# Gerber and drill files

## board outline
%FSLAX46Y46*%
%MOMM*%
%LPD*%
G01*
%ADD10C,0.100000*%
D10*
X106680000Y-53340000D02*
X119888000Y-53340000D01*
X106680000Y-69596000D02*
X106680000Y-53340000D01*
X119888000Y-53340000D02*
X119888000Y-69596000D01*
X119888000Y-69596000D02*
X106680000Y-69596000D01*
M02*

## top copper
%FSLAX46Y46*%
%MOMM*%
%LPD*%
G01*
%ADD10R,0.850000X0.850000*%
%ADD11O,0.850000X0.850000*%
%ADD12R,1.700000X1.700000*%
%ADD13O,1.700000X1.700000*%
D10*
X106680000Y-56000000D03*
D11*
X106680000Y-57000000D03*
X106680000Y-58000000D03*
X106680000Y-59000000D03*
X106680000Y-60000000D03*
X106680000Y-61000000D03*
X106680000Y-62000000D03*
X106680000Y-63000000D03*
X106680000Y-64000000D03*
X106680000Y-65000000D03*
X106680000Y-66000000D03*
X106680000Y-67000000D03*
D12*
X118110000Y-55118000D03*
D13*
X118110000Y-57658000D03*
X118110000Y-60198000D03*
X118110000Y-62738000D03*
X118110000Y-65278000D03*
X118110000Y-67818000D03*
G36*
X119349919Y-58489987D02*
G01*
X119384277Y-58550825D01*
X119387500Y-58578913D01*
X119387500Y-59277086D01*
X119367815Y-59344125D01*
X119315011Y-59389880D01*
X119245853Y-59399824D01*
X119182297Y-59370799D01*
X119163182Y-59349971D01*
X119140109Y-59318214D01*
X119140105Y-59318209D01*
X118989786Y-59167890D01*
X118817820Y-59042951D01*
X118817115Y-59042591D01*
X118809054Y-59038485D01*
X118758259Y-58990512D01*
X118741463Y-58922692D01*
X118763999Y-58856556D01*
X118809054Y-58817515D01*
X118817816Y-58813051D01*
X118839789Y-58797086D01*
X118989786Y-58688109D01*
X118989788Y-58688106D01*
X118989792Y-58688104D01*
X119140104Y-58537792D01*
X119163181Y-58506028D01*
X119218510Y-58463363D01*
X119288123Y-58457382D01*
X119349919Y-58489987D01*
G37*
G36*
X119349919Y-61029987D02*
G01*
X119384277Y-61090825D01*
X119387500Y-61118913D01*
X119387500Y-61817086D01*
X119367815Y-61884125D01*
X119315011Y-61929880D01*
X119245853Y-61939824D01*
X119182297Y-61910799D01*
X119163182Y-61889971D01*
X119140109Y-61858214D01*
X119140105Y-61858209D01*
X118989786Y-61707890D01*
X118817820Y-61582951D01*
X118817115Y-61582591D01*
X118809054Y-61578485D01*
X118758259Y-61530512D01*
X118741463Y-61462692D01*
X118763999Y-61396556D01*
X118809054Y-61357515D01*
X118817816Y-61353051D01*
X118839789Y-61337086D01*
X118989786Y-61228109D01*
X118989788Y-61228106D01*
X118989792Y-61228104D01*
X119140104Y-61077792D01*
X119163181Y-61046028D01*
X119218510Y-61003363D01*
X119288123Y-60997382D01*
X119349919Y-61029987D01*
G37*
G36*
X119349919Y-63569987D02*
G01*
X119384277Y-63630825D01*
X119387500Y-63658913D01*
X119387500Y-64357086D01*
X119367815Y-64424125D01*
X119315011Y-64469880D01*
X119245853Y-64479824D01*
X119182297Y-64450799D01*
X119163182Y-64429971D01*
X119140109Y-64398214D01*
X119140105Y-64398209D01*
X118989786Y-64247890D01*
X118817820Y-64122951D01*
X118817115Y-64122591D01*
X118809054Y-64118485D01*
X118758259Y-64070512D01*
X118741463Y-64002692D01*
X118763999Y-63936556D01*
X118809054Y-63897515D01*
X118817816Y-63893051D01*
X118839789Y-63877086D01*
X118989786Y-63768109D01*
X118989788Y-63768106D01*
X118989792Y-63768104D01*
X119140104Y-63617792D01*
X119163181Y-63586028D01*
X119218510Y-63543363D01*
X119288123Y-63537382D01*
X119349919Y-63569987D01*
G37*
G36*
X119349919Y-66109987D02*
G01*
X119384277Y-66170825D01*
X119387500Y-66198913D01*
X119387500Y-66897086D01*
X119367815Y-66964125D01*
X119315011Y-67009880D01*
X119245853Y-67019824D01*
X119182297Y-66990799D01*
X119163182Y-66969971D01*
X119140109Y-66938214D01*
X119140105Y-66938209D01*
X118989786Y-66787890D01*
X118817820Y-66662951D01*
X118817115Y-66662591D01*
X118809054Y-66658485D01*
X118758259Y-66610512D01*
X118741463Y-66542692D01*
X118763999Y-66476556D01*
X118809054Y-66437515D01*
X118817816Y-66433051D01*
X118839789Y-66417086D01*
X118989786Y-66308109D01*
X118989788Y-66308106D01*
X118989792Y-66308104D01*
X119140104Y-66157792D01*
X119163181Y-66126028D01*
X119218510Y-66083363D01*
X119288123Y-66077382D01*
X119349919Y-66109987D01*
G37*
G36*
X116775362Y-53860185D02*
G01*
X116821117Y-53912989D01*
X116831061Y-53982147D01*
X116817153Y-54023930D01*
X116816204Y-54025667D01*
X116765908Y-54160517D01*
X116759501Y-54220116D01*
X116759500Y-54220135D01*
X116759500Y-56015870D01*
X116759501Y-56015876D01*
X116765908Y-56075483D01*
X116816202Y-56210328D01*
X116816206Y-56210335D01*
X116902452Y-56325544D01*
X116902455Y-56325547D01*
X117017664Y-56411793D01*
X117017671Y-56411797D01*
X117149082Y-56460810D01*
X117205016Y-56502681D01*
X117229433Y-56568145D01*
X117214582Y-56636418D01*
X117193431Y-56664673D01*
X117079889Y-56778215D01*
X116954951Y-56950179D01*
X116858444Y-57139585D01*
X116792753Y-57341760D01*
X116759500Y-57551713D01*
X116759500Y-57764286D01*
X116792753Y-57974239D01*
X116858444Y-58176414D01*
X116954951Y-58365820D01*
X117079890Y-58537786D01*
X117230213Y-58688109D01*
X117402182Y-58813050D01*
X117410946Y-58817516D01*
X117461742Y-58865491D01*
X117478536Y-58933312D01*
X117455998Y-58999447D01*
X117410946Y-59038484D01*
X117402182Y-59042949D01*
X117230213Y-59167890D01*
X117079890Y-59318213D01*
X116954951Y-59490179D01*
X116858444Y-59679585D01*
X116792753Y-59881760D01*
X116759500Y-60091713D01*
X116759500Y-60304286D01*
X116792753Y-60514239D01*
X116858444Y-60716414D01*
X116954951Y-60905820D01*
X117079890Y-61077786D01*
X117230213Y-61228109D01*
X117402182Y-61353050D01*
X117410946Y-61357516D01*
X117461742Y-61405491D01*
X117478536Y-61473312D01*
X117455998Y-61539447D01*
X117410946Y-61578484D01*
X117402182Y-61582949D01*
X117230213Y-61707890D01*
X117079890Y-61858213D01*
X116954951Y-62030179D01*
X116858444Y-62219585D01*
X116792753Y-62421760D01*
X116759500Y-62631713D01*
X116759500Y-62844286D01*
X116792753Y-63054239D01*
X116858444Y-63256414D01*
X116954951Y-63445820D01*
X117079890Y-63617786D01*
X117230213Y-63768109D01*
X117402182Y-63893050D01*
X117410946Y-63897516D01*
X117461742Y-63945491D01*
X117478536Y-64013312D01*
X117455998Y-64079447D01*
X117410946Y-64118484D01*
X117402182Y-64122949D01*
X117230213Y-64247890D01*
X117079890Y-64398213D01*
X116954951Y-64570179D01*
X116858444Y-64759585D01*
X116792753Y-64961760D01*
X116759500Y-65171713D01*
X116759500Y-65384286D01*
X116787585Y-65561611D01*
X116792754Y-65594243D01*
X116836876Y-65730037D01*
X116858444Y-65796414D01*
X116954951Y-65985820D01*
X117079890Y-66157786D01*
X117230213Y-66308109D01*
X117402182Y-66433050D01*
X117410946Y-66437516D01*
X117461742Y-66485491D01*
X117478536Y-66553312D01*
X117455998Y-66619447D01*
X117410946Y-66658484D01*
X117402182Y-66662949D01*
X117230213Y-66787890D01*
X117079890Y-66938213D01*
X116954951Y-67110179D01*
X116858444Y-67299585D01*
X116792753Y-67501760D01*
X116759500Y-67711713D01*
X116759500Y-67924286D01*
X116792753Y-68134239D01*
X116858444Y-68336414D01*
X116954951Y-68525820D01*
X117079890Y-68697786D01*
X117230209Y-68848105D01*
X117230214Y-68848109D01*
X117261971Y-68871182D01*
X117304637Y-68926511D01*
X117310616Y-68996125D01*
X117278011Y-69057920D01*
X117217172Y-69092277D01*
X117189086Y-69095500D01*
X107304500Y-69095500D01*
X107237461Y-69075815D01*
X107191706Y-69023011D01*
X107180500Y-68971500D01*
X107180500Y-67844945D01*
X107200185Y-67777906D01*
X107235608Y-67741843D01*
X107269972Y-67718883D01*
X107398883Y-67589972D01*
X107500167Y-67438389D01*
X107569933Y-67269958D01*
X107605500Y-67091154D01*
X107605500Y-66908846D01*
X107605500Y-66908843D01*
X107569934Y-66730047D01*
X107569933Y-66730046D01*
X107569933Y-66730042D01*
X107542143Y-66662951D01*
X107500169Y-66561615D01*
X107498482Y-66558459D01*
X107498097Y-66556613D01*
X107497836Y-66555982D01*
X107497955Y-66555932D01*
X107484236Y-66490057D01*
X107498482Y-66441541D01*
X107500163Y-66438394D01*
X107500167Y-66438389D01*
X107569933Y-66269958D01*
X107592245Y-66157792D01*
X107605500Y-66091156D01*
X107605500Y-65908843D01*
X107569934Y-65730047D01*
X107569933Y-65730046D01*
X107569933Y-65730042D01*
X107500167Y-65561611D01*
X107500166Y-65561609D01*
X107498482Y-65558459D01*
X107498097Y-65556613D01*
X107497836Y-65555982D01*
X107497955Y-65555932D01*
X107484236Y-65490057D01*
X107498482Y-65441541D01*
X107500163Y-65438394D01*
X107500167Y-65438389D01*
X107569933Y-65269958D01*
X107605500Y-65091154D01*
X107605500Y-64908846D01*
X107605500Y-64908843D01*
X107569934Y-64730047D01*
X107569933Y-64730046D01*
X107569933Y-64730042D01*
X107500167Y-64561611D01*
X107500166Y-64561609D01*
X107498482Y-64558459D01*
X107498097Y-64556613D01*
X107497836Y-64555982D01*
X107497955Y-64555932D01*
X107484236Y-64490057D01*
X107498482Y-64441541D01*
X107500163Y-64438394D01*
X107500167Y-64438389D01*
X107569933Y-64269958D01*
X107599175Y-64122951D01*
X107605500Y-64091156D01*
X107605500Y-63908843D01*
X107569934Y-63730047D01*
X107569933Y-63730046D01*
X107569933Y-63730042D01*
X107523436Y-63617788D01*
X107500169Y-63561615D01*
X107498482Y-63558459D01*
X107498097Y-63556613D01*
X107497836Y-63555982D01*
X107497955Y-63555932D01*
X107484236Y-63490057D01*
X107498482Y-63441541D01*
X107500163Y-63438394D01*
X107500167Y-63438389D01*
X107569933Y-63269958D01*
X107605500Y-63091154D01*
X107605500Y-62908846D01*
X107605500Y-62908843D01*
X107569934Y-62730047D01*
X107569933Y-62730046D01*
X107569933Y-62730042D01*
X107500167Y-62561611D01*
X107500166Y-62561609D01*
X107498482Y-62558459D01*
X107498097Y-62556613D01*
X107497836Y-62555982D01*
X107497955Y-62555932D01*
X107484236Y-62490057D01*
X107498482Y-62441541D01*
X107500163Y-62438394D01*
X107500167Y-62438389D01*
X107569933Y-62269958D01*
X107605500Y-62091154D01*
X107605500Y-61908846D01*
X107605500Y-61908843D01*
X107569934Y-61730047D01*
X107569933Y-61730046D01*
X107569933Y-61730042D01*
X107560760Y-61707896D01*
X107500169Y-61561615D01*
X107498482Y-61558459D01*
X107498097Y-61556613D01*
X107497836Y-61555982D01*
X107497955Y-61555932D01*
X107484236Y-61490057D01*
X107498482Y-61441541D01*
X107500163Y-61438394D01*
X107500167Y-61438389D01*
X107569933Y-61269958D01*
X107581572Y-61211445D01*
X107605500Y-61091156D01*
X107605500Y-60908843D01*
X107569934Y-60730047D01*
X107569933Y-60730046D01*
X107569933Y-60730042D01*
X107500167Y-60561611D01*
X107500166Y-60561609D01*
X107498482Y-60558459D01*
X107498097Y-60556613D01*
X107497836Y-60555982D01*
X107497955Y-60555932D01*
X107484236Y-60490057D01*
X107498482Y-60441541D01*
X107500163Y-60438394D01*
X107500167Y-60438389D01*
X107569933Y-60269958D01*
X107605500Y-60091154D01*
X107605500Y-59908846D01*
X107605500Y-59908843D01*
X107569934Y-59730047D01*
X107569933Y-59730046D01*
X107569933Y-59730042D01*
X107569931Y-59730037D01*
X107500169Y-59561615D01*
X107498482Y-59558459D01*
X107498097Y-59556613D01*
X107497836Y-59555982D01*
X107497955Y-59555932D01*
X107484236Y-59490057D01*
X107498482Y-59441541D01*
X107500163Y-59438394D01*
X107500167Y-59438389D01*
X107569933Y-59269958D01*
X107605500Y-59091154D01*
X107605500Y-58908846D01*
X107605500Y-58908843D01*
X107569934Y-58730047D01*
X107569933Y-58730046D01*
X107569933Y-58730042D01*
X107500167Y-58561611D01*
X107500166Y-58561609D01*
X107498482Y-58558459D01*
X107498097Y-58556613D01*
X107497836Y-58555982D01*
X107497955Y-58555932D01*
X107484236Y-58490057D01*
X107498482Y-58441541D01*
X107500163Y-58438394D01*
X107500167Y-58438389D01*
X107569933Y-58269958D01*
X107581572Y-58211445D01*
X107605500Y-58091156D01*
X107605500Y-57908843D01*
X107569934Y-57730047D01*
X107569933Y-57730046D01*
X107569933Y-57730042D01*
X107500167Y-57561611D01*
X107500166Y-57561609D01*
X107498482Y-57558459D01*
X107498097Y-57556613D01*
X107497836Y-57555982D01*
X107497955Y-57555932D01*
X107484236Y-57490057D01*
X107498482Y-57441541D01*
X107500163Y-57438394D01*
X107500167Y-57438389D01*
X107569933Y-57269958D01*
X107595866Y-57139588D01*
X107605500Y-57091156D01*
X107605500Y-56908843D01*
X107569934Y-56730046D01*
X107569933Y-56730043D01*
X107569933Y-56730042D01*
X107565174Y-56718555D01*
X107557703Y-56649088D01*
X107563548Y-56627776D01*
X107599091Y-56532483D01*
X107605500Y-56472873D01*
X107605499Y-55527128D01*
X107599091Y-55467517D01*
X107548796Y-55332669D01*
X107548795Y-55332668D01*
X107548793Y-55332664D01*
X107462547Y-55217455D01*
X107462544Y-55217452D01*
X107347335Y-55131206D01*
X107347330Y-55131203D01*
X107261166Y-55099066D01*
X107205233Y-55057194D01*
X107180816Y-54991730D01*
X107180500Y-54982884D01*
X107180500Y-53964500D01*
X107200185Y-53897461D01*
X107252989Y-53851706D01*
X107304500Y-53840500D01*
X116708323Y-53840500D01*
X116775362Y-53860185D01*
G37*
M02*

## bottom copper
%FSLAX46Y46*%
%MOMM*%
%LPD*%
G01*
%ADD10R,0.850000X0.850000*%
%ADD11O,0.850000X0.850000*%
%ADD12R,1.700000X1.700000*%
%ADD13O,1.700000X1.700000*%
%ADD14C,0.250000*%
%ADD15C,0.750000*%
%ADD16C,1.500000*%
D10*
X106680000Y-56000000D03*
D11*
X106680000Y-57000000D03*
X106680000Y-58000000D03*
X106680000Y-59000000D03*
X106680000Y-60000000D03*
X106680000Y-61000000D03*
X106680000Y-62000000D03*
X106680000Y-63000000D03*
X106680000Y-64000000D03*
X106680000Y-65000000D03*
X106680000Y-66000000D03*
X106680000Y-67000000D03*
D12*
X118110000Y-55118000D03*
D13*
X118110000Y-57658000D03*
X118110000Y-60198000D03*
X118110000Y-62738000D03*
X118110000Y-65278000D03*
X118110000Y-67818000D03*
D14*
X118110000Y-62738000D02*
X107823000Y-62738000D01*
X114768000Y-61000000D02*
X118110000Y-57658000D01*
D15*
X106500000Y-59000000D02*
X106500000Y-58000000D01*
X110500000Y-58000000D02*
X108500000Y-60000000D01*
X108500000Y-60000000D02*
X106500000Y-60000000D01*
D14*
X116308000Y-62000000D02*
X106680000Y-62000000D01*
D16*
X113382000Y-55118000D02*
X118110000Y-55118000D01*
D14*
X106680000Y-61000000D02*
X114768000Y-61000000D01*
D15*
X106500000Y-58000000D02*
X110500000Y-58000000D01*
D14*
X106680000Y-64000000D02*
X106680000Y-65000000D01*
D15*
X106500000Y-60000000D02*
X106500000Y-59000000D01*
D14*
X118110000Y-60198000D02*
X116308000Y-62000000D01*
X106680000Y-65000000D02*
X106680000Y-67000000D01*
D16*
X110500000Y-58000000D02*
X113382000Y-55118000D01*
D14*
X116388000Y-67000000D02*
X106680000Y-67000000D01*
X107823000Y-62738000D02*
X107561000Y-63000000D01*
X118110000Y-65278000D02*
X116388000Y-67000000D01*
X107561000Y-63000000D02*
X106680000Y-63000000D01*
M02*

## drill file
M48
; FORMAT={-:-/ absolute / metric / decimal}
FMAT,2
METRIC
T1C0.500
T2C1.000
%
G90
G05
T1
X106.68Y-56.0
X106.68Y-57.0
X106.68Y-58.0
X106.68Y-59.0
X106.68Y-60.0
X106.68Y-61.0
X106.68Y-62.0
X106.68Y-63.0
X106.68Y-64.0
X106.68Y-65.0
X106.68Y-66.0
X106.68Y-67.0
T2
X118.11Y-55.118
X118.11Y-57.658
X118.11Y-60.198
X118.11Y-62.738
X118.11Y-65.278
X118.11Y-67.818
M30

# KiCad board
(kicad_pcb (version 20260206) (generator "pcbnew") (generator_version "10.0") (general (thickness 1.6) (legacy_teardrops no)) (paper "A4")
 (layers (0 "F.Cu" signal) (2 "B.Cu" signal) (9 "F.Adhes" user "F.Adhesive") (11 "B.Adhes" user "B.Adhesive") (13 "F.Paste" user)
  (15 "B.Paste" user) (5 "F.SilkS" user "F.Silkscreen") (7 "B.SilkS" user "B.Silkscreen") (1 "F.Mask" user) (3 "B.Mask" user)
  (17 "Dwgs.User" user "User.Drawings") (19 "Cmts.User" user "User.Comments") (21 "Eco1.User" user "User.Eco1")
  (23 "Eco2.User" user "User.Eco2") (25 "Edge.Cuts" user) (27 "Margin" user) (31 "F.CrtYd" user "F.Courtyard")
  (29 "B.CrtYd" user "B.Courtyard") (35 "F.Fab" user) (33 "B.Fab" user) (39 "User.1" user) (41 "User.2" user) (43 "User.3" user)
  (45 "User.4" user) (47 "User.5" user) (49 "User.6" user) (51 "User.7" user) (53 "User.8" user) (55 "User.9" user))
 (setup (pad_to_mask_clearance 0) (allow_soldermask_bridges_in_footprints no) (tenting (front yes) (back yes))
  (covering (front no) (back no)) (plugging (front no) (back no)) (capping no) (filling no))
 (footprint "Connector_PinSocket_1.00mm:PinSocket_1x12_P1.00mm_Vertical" (layer "F.Cu") (at 106.68 56)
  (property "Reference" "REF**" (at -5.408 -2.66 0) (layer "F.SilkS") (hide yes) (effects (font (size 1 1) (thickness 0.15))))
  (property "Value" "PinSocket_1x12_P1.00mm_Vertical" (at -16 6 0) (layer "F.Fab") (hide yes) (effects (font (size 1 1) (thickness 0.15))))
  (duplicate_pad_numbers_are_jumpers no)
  (pad "1" thru_hole rect (at 0 0) (size 0.85 0.85) (drill 0.5) (layers "*.Cu" "*.Mask") (remove_unused_layers no))
  (pad "2" thru_hole oval (at 0 1) (size 0.85 0.85) (drill 0.5) (layers "*.Cu" "*.Mask") (remove_unused_layers no))
  (pad "3" thru_hole oval (at 0 2) (size 0.85 0.85) (drill 0.5) (layers "*.Cu" "*.Mask") (remove_unused_layers no))
  (pad "4" thru_hole oval (at 0 3) (size 0.85 0.85) (drill 0.5) (layers "*.Cu" "*.Mask") (remove_unused_layers no))
  (pad "5" thru_hole oval (at 0 4) (size 0.85 0.85) (drill 0.5) (layers "*.Cu" "*.Mask") (remove_unused_layers no))
  (pad "6" thru_hole oval (at 0 5) (size 0.85 0.85) (drill 0.5) (layers "*.Cu" "*.Mask") (remove_unused_layers no))
  (pad "7" thru_hole oval (at 0 6) (size 0.85 0.85) (drill 0.5) (layers "*.Cu" "*.Mask") (remove_unused_layers no))
  (pad "8" thru_hole oval (at 0 7) (size 0.85 0.85) (drill 0.5) (layers "*.Cu" "*.Mask") (remove_unused_layers no))
  (pad "9" thru_hole oval (at 0 8) (size 0.85 0.85) (drill 0.5) (layers "*.Cu" "*.Mask") (remove_unused_layers no))
  (pad "10" thru_hole oval (at 0 9) (size 0.85 0.85) (drill 0.5) (layers "*.Cu" "*.Mask") (remove_unused_layers no))
  (pad "11" thru_hole oval (at 0 10) (size 0.85 0.85) (drill 0.5) (layers "*.Cu" "*.Mask") (remove_unused_layers no))
  (pad "12" thru_hole oval (at 0 11) (size 0.85 0.85) (drill 0.5) (layers "*.Cu" "*.Mask") (remove_unused_layers no)))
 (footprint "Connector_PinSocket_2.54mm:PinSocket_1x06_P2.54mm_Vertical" (layer "F.Cu") (at 118.11 55.118)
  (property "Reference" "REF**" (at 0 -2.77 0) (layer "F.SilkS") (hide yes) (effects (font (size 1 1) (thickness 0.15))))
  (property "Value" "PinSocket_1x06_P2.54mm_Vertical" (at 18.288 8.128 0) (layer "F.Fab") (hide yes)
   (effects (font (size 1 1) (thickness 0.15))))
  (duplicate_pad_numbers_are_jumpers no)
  (pad "1" thru_hole rect (at 0 0) (size 1.7 1.7) (drill 1) (layers "*.Cu" "*.Mask") (remove_unused_layers no))
  (pad "2" thru_hole oval (at 0 2.54) (size 1.7 1.7) (drill 1) (layers "*.Cu" "*.Mask") (remove_unused_layers no))
  (pad "3" thru_hole oval (at 0 5.08) (size 1.7 1.7) (drill 1) (layers "*.Cu" "*.Mask") (remove_unused_layers no))
  (pad "4" thru_hole oval (at 0 7.62) (size 1.7 1.7) (drill 1) (layers "*.Cu" "*.Mask") (remove_unused_layers no))
  (pad "5" thru_hole oval (at 0 10.16) (size 1.7 1.7) (drill 1) (layers "*.Cu" "*.Mask") (remove_unused_layers no))
  (pad "6" thru_hole oval (at 0 12.7) (size 1.7 1.7) (drill 1) (layers "*.Cu" "*.Mask") (remove_unused_layers no)))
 (gr_line (start 106.68 53.34) (end 119.888 53.34) (stroke (width 0.1) (type default)) (layer "Edge.Cuts"))
 (gr_line (start 106.68 69.596) (end 106.68 53.34) (stroke (width 0.1) (type default)) (layer "Edge.Cuts"))
 (gr_line (start 119.888 53.34) (end 119.888 69.596) (stroke (width 0.1) (type default)) (layer "Edge.Cuts"))
 (gr_line (start 119.888 69.596) (end 106.68 69.596) (stroke (width 0.1) (type default)) (layer "Edge.Cuts"))
 (segment (start 118.11 62.738) (end 107.823 62.738) (width 0.25) (layer "B.Cu") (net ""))
 (segment (start 114.768 61) (end 118.11 57.658) (width 0.25) (layer "B.Cu") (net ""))
 (segment (start 106.5 59) (end 106.5 58) (width 0.75) (layer "B.Cu") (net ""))
 (segment (start 110.5 58) (end 108.5 60) (width 0.75) (layer "B.Cu") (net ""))
 (segment (start 108.5 60) (end 106.5 60) (width 0.75) (layer "B.Cu") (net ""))
 (segment (start 116.308 62) (end 106.68 62) (width 0.25) (layer "B.Cu") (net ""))
 (segment (start 113.382 55.118) (end 118.11 55.118) (width 1.5) (layer "B.Cu") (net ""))
 (segment (start 106.68 61) (end 114.768 61) (width 0.25) (layer "B.Cu") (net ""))
 (segment (start 106.5 58) (end 110.5 58) (width 0.75) (layer "B.Cu") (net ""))
 (segment (start 106.68 64) (end 106.68 65) (width 0.25) (layer "B.Cu") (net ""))
 (segment (start 106.5 60) (end 106.5 59) (width 0.75) (layer "B.Cu") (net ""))
 (segment (start 118.11 60.198) (end 116.308 62) (width 0.25) (layer "B.Cu") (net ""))
 (segment (start 106.68 65) (end 106.68 67) (width 0.25) (layer "B.Cu") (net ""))
 (segment (start 110.5 58) (end 113.382 55.118) (width 1.5) (layer "B.Cu") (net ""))
 (segment (start 116.388 67) (end 106.68 67) (width 0.25) (layer "B.Cu") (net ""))
 (segment (start 107.823 62.738) (end 107.561 63) (width 0.25) (layer "B.Cu") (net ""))
 (segment (start 118.11 65.278) (end 116.388 67) (width 0.25) (layer "B.Cu") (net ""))
 (segment (start 107.561 63) (end 106.68 63) (width 0.25) (layer "B.Cu") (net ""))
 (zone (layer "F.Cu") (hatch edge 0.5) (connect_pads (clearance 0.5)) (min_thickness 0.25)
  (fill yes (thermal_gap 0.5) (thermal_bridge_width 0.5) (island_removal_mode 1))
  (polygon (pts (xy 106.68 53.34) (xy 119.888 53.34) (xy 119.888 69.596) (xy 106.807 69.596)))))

